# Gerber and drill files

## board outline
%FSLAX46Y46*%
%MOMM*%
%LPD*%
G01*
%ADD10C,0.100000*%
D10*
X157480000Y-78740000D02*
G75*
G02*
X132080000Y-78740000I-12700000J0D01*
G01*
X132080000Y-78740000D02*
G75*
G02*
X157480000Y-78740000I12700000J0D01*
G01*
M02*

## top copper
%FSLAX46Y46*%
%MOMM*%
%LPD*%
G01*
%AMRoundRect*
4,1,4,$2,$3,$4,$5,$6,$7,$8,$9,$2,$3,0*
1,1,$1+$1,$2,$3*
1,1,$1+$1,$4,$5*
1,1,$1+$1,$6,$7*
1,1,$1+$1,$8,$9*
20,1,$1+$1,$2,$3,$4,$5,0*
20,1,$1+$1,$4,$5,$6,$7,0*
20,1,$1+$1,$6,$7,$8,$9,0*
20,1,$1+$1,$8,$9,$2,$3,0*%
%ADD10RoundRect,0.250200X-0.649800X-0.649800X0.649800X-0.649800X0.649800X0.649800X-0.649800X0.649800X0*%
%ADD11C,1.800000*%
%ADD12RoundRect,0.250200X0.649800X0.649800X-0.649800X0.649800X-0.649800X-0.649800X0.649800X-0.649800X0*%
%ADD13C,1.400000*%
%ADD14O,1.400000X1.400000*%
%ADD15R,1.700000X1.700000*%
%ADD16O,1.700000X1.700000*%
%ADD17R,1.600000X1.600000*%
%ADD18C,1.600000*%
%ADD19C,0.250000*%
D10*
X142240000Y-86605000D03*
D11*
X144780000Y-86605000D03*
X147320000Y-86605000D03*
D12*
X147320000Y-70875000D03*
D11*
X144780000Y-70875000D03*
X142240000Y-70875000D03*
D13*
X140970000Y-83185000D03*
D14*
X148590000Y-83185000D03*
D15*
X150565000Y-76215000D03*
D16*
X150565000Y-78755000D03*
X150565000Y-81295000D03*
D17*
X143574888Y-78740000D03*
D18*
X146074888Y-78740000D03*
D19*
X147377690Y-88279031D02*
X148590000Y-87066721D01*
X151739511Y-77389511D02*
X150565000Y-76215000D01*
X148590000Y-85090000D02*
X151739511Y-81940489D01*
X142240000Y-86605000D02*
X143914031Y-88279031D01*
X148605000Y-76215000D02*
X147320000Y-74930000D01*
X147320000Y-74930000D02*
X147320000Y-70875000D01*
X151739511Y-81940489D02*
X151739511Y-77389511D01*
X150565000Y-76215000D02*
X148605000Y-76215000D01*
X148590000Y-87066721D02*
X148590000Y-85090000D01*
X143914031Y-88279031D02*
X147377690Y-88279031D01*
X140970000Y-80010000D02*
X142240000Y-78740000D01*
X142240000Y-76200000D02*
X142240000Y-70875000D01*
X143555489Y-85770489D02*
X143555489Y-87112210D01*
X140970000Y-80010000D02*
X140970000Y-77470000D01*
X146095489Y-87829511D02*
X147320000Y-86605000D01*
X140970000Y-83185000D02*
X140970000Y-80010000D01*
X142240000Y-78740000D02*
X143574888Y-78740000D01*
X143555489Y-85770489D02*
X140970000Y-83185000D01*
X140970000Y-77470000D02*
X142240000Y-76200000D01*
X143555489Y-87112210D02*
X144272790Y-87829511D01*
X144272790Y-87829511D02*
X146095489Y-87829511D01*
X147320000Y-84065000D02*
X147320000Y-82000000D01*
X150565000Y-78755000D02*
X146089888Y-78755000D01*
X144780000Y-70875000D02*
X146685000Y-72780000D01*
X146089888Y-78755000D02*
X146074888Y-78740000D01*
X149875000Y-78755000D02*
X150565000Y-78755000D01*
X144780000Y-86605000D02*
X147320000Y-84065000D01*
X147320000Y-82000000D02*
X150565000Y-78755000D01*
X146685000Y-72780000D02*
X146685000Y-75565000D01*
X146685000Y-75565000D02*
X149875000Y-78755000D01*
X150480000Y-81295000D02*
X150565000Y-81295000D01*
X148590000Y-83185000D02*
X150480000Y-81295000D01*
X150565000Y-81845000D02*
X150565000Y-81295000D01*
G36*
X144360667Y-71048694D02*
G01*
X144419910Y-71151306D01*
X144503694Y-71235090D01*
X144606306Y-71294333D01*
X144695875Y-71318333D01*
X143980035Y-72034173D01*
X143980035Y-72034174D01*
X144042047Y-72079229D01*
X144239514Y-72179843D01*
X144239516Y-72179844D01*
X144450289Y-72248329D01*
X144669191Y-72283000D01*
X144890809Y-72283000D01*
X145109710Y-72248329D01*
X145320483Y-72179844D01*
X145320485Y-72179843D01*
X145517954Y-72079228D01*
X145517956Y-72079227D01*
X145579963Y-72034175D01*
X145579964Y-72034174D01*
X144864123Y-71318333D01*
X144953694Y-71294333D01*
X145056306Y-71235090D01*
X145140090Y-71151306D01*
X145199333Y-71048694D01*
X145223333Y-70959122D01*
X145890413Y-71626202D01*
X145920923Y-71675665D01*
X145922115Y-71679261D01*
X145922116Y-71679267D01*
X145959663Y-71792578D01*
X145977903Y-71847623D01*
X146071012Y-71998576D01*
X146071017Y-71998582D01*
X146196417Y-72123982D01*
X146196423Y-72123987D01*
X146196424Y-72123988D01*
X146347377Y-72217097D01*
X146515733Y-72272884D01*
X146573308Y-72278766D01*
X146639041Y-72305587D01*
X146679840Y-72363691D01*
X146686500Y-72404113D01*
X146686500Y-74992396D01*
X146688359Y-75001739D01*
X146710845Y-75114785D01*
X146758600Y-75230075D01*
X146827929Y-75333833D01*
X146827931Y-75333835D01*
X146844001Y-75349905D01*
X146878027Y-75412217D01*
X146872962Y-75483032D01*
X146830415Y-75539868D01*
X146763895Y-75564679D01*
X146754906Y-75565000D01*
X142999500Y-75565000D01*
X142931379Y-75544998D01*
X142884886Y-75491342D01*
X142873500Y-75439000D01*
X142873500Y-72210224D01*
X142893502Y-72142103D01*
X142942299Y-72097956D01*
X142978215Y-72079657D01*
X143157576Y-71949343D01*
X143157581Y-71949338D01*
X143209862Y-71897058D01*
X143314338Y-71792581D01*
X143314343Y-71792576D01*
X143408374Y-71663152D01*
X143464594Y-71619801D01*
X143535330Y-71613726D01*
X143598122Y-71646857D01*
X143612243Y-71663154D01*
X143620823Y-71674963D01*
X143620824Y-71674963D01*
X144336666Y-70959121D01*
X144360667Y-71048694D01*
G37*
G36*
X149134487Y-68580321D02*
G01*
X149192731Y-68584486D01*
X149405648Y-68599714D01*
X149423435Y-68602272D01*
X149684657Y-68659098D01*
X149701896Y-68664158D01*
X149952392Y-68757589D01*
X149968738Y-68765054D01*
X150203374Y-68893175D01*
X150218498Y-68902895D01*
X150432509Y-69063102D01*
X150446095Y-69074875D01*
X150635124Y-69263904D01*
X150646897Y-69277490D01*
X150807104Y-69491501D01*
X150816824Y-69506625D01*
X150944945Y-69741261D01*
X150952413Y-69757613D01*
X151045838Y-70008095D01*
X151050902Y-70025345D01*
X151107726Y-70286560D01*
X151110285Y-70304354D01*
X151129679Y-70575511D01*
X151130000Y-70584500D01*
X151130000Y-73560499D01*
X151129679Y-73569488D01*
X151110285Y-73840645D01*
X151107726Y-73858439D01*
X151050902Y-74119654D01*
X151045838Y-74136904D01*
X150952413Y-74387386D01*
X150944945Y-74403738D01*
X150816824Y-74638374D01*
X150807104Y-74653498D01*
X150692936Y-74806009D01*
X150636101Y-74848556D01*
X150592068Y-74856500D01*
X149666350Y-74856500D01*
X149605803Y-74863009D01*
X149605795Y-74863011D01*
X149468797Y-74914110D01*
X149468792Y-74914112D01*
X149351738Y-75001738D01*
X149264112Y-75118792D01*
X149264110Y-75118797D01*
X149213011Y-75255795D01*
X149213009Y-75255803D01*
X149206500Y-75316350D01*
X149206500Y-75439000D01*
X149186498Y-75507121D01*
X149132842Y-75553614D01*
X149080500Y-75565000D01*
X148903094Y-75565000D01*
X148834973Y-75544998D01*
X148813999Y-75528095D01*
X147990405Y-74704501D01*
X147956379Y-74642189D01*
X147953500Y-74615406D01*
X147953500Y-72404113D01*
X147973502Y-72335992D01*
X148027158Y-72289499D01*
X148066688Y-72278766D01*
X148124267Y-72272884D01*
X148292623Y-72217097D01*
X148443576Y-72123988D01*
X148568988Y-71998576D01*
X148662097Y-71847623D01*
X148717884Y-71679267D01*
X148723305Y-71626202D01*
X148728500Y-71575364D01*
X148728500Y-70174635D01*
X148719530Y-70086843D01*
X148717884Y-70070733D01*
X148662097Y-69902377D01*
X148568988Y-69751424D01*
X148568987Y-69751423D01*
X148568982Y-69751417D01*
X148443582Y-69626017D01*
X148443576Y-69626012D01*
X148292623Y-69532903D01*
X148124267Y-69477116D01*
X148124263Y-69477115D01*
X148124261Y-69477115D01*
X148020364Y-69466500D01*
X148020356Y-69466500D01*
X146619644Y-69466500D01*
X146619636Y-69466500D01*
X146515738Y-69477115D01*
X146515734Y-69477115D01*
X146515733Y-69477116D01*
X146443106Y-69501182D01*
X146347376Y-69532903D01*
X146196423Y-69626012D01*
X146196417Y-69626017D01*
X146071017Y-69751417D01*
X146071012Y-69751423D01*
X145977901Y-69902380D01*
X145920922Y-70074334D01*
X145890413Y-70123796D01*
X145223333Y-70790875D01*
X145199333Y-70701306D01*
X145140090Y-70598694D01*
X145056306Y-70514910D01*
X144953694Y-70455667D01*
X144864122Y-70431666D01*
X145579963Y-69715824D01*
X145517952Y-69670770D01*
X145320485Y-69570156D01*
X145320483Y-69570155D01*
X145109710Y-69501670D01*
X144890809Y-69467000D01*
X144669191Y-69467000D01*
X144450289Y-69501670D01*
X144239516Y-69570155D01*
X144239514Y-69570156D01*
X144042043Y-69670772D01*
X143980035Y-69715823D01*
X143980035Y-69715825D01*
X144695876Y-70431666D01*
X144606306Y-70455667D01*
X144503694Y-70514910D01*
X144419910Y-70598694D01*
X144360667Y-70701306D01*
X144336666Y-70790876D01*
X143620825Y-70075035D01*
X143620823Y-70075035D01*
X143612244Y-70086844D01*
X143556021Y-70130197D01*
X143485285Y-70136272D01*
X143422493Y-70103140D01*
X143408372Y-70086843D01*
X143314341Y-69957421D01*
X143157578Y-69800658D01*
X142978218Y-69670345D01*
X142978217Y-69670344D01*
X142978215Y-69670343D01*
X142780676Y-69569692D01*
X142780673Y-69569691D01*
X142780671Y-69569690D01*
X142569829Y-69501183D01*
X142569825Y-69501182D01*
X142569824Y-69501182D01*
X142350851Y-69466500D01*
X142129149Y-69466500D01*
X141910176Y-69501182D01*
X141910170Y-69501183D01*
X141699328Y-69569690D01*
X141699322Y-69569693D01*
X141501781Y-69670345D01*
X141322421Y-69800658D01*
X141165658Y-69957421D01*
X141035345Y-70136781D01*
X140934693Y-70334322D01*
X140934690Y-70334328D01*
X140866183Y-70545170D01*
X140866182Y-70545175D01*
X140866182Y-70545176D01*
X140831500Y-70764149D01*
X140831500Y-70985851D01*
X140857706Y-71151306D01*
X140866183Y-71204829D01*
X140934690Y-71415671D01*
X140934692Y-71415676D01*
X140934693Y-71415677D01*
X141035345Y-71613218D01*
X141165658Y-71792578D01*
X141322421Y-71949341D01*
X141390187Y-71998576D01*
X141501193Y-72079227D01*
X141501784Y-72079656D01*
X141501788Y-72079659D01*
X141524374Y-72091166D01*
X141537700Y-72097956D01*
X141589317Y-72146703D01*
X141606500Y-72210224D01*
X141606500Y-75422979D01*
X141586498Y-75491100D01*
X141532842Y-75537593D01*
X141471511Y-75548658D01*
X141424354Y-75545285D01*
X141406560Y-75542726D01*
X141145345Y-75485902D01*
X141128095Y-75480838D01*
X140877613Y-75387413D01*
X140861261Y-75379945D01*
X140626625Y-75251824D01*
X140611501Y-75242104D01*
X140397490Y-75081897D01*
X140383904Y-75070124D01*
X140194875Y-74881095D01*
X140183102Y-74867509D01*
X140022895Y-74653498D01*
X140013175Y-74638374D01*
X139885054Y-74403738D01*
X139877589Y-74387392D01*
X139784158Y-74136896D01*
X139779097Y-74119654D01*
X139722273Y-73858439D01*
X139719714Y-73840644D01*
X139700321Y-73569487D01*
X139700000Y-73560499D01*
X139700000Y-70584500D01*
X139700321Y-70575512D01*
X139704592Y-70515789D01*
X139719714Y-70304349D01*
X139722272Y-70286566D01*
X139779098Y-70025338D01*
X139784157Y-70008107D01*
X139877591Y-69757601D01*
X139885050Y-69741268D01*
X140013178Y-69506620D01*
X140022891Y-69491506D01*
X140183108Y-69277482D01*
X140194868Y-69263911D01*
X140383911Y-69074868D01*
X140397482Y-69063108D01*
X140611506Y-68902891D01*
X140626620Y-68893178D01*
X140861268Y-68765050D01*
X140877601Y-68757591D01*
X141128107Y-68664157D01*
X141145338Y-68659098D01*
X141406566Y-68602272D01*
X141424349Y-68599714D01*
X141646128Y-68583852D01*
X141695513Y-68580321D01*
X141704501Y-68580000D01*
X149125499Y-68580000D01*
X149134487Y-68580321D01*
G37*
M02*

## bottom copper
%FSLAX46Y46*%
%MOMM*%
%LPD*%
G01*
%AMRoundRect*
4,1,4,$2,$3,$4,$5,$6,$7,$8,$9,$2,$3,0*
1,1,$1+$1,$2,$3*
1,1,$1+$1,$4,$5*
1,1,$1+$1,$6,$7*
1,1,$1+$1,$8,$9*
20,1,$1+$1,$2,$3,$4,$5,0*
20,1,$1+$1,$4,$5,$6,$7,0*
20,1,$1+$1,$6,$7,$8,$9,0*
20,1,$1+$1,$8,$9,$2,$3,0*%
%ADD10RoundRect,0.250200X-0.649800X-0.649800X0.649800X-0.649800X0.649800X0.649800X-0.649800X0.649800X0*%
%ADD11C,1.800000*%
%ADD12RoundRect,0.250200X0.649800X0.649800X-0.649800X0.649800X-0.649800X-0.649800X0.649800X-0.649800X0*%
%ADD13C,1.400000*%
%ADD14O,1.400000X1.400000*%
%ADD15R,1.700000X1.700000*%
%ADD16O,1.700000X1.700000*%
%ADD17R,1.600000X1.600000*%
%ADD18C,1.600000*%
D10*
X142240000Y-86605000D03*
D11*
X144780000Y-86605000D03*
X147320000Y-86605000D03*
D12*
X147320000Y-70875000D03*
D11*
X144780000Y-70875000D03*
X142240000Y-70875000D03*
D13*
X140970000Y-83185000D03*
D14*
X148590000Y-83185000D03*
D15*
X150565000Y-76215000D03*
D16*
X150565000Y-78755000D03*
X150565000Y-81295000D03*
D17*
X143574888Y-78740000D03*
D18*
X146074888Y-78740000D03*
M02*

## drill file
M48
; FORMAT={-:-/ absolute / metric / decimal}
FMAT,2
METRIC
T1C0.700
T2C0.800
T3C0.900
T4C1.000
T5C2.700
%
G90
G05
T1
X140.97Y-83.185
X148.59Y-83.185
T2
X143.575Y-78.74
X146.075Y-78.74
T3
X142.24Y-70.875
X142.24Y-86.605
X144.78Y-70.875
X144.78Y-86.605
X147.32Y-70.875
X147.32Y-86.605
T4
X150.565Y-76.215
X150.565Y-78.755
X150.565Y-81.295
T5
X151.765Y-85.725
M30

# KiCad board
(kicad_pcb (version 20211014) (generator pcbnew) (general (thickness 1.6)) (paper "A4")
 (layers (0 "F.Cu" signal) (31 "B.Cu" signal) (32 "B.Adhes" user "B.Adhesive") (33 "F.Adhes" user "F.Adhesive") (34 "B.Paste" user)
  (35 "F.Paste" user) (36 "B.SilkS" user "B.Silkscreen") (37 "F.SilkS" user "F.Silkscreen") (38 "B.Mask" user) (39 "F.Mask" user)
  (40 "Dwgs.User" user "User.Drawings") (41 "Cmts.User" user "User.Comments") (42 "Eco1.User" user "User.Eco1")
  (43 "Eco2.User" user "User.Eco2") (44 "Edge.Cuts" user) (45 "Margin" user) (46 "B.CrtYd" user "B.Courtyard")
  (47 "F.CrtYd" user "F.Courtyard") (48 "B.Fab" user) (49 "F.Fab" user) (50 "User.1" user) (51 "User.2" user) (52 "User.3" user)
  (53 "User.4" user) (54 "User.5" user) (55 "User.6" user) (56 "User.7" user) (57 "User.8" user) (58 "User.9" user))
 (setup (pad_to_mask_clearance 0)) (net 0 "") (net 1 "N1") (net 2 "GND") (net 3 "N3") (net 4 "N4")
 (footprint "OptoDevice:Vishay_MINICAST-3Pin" (layer "F.Cu") (at 142.24 86.605)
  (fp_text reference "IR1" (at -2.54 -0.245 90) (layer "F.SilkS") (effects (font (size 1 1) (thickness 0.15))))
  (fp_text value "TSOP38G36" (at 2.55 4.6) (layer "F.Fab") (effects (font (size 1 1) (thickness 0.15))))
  (pad "1" thru_hole roundrect (at 0 0) (size 1.8 1.8) (drill 0.9) (layers *.Cu *.Mask) (roundrect_rratio 0.139) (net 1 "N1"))
  (pad "2" thru_hole circle (at 2.54 0) (size 1.8 1.8) (drill 0.9) (layers *.Cu *.Mask) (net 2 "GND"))
  (pad "3" thru_hole circle (at 5.08 0) (size 1.8 1.8) (drill 0.9) (layers *.Cu *.Mask) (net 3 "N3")))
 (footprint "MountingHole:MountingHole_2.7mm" (layer "F.Cu") (at 151.765 85.725)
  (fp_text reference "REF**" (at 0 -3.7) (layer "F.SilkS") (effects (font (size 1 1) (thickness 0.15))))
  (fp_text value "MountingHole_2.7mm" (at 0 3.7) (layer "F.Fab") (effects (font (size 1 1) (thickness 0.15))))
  (pad "" np_thru_hole circle (at 0 0) (size 2.7 2.7) (drill 2.7) (layers *.Cu *.Mask)))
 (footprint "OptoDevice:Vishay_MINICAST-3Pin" (layer "F.Cu") (at 147.32 70.875 180)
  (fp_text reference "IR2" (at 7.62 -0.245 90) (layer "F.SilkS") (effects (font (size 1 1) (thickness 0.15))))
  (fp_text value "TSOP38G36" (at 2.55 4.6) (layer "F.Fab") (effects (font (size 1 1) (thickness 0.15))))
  (pad "1" thru_hole roundrect (at 0 0 180) (size 1.8 1.8) (drill 0.9) (layers *.Cu *.Mask) (roundrect_rratio 0.139) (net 1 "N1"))
  (pad "2" thru_hole circle (at 2.54 0 180) (size 1.8 1.8) (drill 0.9) (layers *.Cu *.Mask) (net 2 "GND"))
  (pad "3" thru_hole circle (at 5.08 0 180) (size 1.8 1.8) (drill 0.9) (layers *.Cu *.Mask) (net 3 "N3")))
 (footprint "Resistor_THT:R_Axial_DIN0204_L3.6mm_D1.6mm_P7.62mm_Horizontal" (layer "F.Cu") (at 140.97 83.185)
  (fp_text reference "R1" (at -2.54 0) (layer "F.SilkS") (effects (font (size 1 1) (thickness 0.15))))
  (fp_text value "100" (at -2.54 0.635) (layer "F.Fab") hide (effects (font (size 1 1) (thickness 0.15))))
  (pad "1" thru_hole circle (at 0 0) (size 1.4 1.4) (drill 0.7) (layers *.Cu *.Mask) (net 3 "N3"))
  (pad "2" thru_hole oval (at 7.62 0) (size 1.4 1.4) (drill 0.7) (layers *.Cu *.Mask) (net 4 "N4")))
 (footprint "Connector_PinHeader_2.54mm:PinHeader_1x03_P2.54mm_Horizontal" (layer "F.Cu") (at 150.565 76.215)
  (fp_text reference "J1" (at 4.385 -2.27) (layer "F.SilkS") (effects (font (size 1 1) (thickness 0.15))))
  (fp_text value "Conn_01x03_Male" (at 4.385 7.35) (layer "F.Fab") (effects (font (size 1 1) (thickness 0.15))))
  (pad "1" thru_hole rect (at 0 0) (size 1.7 1.7) (drill 1) (layers *.Cu *.Mask) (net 1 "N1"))
  (pad "2" thru_hole oval (at 0 2.54) (size 1.7 1.7) (drill 1) (layers *.Cu *.Mask) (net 2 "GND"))
  (pad "3" thru_hole oval (at 0 5.08) (size 1.7 1.7) (drill 1) (layers *.Cu *.Mask) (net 4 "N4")))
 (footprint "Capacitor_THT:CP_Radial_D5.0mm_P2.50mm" (layer "F.Cu") (at 143.574888 78.74)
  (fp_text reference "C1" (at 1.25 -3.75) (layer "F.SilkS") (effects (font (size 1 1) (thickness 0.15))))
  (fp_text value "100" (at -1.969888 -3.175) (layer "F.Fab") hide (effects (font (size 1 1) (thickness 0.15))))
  (pad "1" thru_hole rect (at 0 0) (size 1.6 1.6) (drill 0.8) (layers *.Cu *.Mask) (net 3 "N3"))
  (pad "2" thru_hole circle (at 2.5 0) (size 1.6 1.6) (drill 0.8) (layers *.Cu *.Mask) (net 2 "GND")))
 (gr_circle (center 144.78 78.74) (end 157.48 78.74) (layer "Edge.Cuts") (width 0.1) (fill none))
 (segment (start 147.37769 88.279031) (end 148.59 87.066721) (width 0.25) (layer "F.Cu") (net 1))
 (segment (start 151.739511 77.389511) (end 150.565 76.215) (width 0.25) (layer "F.Cu") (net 1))
 (segment (start 148.59 85.09) (end 151.739511 81.940489) (width 0.25) (layer "F.Cu") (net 1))
 (segment (start 142.24 86.605) (end 143.914031 88.279031) (width 0.25) (layer "F.Cu") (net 1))
 (segment (start 148.605 76.215) (end 147.32 74.93) (width 0.25) (layer "F.Cu") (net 1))
 (segment (start 147.32 74.93) (end 147.32 70.875) (width 0.25) (layer "F.Cu") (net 1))
 (segment (start 151.739511 81.940489) (end 151.739511 77.389511) (width 0.25) (layer "F.Cu") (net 1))
 (segment (start 150.565 76.215) (end 148.605 76.215) (width 0.25) (layer "F.Cu") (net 1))
 (segment (start 148.59 87.066721) (end 148.59 85.09) (width 0.25) (layer "F.Cu") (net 1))
 (segment (start 143.914031 88.279031) (end 147.37769 88.279031) (width 0.25) (layer "F.Cu") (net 1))
 (segment (start 140.97 80.01) (end 142.24 78.74) (width 0.25) (layer "F.Cu") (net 3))
 (segment (start 142.24 76.2) (end 142.24 70.875) (width 0.25) (layer "F.Cu") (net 3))
 (segment (start 143.555489 85.770489) (end 143.555489 87.11221) (width 0.25) (layer "F.Cu") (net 3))
 (segment (start 140.97 80.01) (end 140.97 77.47) (width 0.25) (layer "F.Cu") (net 3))
 (segment (start 146.095489 87.829511) (end 147.32 86.605) (width 0.25) (layer "F.Cu") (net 3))
 (segment (start 140.97 83.185) (end 140.97 80.01) (width 0.25) (layer "F.Cu") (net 3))
 (segment (start 142.24 78.74) (end 143.574888 78.74) (width 0.25) (layer "F.Cu") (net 3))
 (segment (start 143.555489 85.770489) (end 140.97 83.185) (width 0.25) (layer "F.Cu") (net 3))
 (segment (start 140.97 77.47) (end 142.24 76.2) (width 0.25) (layer "F.Cu") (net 3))
 (segment (start 143.555489 87.11221) (end 144.27279 87.829511) (width 0.25) (layer "F.Cu") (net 3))
 (segment (start 144.27279 87.829511) (end 146.095489 87.829511) (width 0.25) (layer "F.Cu") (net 3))
 (segment (start 147.32 84.065) (end 147.32 82) (width 0.25) (layer "F.Cu") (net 2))
 (segment (start 150.565 78.755) (end 146.089888 78.755) (width 0.25) (layer "F.Cu") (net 2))
 (segment (start 144.78 70.875) (end 146.685 72.78) (width 0.25) (layer "F.Cu") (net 2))
 (segment (start 146.089888 78.755) (end 146.074888 78.74) (width 0.25) (layer "F.Cu") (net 2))
 (segment (start 149.875 78.755) (end 150.565 78.755) (width 0.25) (layer "F.Cu") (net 2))
 (segment (start 144.78 86.605) (end 147.32 84.065) (width 0.25) (layer "F.Cu") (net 2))
 (segment (start 147.32 82) (end 150.565 78.755) (width 0.25) (layer "F.Cu") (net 2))
 (segment (start 146.685 72.78) (end 146.685 75.565) (width 0.25) (layer "F.Cu") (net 2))
 (segment (start 146.685 75.565) (end 149.875 78.755) (width 0.25) (layer "F.Cu") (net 2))
 (segment (start 150.48 81.295) (end 150.565 81.295) (width 0.25) (layer "F.Cu") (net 4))
 (segment (start 148.59 83.185) (end 150.48 81.295) (width 0.25) (layer "F.Cu") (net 4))
 (segment (start 150.565 81.845) (end 150.565 81.295) (width 0.25) (layer "F.Cu") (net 4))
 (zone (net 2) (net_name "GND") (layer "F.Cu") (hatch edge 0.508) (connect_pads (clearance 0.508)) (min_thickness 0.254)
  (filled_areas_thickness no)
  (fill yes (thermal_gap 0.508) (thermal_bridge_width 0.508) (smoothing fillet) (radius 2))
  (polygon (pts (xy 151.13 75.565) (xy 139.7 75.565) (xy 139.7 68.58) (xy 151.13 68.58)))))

